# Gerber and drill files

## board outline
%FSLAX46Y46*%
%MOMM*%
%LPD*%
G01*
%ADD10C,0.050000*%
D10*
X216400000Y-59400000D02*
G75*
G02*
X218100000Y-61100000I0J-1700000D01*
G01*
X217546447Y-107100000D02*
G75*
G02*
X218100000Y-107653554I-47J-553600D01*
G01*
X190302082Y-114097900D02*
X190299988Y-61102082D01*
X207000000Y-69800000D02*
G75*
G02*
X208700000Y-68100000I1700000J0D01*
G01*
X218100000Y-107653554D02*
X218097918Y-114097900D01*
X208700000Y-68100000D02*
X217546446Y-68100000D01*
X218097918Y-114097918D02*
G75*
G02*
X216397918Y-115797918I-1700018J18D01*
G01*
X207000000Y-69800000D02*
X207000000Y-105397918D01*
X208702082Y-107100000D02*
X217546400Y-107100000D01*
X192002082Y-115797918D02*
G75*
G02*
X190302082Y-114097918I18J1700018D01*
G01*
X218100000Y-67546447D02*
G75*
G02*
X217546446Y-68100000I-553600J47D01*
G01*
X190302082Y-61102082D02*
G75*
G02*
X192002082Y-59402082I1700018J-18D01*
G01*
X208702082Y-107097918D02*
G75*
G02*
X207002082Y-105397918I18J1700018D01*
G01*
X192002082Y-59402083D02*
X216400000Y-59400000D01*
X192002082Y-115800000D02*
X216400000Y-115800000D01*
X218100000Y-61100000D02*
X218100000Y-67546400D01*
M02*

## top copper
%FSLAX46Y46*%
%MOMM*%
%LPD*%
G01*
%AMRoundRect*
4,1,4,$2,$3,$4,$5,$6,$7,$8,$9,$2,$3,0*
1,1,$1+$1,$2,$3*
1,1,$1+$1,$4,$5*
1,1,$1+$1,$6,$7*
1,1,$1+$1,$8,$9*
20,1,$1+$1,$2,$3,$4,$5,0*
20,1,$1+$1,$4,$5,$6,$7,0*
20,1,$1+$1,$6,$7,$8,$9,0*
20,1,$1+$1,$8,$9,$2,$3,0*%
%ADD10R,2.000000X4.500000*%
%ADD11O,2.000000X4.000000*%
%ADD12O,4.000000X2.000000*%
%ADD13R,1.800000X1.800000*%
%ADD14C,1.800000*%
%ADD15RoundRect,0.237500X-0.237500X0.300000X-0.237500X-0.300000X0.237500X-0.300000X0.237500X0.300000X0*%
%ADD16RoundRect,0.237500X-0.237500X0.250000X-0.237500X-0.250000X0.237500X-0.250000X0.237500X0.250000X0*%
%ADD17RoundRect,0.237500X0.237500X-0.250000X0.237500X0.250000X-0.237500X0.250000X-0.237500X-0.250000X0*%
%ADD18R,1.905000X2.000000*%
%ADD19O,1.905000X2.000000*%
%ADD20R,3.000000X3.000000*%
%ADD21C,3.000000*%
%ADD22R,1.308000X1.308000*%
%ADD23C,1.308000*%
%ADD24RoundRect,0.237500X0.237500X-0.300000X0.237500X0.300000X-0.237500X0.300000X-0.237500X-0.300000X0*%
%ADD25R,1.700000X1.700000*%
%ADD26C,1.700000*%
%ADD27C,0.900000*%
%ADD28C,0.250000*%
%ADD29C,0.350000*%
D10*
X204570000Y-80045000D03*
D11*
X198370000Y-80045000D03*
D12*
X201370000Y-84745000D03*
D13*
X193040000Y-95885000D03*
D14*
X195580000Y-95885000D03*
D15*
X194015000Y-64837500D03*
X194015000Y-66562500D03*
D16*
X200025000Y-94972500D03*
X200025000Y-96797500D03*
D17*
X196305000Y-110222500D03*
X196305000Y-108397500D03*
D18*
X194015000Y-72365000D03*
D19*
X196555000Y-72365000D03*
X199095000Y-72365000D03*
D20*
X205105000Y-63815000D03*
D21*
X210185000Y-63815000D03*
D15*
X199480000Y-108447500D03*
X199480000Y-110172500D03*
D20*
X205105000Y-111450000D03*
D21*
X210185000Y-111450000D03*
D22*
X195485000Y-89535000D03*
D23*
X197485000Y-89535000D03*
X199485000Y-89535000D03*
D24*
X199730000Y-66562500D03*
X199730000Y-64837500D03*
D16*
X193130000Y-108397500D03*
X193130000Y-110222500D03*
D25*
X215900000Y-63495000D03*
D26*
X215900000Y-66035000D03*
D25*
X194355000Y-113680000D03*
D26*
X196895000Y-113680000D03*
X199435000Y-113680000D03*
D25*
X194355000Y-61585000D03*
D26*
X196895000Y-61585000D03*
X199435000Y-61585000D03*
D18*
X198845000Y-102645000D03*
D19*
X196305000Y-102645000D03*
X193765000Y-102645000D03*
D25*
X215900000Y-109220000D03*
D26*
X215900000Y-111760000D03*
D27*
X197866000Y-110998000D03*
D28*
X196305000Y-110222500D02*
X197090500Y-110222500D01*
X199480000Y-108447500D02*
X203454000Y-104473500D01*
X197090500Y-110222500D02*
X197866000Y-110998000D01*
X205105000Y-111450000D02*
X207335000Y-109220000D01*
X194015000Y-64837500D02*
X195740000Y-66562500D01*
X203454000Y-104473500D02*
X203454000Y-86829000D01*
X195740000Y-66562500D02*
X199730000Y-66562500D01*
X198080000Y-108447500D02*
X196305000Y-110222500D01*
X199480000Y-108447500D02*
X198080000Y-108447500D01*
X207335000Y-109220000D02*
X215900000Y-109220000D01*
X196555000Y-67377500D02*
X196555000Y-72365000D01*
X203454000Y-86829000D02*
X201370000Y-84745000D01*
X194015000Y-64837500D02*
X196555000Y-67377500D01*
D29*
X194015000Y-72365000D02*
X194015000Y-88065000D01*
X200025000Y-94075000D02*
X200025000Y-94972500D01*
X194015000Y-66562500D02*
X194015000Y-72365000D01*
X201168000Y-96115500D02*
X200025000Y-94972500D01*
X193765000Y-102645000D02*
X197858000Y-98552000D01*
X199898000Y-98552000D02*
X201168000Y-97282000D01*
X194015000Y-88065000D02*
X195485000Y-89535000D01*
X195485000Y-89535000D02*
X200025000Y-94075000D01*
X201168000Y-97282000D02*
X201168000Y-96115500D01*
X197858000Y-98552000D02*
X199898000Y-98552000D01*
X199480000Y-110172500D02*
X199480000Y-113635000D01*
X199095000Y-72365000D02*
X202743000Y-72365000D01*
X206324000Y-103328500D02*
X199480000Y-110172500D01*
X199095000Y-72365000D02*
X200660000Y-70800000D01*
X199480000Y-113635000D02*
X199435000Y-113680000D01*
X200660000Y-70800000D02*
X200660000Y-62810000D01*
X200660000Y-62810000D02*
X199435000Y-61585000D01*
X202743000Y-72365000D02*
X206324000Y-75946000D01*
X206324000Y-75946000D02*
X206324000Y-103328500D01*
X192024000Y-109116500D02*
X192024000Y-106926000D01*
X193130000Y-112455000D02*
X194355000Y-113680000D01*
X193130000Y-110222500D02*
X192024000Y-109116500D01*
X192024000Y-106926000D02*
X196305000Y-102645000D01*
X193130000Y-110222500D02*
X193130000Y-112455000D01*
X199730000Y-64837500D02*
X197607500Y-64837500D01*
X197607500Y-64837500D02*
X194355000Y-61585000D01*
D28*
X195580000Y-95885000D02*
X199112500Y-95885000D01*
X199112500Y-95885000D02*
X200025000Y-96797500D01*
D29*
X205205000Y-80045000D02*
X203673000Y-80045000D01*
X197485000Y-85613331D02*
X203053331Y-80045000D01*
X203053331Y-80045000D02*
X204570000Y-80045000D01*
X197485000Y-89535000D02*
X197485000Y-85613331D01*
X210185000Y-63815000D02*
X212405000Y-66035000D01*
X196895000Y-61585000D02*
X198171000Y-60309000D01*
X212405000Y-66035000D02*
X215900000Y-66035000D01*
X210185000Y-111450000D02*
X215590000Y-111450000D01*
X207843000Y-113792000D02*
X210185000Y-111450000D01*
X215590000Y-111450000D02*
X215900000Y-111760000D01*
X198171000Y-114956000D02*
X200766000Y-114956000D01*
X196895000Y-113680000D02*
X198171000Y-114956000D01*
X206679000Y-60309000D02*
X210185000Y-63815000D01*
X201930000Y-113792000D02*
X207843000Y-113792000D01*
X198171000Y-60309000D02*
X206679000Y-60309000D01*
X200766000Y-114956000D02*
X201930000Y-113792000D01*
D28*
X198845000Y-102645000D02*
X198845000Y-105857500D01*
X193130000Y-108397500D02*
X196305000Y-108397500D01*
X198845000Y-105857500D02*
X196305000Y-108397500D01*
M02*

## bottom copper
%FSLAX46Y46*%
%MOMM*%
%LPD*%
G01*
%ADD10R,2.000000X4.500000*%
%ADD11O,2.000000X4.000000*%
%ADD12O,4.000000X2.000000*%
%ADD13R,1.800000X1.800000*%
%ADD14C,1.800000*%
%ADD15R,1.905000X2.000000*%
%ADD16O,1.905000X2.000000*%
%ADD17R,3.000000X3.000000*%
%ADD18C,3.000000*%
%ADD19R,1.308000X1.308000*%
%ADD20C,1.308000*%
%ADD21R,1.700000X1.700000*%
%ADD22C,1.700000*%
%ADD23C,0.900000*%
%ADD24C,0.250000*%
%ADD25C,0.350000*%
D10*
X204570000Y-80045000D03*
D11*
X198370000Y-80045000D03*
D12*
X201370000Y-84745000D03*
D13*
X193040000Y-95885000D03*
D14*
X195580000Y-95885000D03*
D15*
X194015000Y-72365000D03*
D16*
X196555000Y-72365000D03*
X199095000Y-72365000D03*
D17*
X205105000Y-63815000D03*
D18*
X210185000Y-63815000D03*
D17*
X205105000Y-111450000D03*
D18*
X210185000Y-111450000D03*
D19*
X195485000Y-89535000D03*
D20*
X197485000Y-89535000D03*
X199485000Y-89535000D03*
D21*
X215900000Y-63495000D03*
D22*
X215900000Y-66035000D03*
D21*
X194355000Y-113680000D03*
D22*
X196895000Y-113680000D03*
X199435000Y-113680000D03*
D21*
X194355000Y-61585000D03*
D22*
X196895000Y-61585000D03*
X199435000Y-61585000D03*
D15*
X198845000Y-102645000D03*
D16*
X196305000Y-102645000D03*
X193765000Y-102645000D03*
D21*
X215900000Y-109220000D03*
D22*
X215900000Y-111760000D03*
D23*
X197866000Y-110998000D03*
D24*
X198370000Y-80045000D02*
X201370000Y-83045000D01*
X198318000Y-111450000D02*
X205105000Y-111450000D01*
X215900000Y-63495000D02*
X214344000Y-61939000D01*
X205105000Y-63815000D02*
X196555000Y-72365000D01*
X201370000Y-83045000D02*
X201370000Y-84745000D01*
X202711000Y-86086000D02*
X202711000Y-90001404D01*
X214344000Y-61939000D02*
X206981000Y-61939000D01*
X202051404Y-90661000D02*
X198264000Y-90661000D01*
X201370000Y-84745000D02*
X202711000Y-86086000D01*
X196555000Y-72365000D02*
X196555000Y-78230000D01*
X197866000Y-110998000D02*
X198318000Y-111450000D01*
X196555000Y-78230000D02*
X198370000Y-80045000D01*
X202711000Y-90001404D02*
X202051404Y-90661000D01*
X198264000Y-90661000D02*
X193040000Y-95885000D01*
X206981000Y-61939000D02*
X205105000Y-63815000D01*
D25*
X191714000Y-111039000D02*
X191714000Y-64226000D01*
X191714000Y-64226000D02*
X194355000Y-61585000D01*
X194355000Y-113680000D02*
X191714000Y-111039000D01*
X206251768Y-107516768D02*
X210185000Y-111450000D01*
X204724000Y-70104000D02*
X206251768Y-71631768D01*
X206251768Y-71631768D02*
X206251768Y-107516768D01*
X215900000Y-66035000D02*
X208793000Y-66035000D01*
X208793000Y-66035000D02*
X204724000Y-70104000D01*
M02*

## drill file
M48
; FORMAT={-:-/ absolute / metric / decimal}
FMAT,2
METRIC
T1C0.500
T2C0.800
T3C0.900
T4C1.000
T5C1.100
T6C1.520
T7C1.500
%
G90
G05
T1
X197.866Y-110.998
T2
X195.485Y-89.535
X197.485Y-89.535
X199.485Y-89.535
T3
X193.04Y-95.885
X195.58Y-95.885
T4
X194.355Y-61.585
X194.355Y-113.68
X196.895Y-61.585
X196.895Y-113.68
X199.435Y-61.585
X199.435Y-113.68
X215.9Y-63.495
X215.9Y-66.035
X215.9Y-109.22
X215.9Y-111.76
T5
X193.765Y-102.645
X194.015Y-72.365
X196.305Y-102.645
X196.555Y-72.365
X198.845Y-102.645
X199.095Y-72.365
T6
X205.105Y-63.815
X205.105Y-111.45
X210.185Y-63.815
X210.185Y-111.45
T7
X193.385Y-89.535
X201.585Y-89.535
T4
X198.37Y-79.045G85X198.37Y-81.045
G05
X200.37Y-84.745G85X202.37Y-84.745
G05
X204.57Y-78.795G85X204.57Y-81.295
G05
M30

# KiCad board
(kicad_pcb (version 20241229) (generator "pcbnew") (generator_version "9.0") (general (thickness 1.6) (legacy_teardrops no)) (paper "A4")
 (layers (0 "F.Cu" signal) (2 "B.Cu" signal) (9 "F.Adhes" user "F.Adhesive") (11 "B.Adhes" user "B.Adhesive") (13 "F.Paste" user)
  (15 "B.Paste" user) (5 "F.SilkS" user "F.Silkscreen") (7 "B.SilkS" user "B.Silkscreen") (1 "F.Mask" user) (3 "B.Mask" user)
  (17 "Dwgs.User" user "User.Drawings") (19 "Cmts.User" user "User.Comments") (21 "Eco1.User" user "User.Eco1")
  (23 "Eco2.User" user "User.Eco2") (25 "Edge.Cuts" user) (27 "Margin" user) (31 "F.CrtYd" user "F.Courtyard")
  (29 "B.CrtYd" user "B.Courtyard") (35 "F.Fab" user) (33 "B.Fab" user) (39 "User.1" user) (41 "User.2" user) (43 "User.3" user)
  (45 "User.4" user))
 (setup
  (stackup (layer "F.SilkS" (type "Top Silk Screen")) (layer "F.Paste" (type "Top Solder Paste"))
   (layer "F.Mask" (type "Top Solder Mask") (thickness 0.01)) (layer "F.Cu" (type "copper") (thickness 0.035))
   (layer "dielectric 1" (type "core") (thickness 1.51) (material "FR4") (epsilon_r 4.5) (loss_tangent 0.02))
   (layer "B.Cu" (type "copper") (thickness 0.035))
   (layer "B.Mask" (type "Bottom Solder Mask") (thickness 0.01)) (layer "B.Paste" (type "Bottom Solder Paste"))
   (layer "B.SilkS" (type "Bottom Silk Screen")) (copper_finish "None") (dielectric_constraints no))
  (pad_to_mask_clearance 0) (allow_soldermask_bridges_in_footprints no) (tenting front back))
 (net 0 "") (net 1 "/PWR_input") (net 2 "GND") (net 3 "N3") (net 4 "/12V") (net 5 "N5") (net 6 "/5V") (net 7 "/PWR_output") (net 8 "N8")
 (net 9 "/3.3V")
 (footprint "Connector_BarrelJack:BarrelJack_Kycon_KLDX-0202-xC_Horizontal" (layer "F.Cu") (at 204.57 80.045)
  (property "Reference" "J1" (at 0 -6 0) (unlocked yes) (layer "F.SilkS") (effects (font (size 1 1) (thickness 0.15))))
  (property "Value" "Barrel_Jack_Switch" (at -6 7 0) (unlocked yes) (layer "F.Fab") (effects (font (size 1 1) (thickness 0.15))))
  (pad "1" thru_hole rect (at 0 0) (size 2 4.5) (drill oval 1 3.5) (layers "*.Cu" "*.Mask") (remove_unused_layers no) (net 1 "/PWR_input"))
  (pad "2" thru_hole oval (at -6.2 0) (size 2 4) (drill oval 1 3) (layers "*.Cu" "*.Mask") (remove_unused_layers no) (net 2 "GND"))
  (pad "3" thru_hole oval (at -3.2 4.7 90) (size 2 4) (drill oval 1 3) (layers "*.Cu" "*.Mask") (remove_unused_layers no) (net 2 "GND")))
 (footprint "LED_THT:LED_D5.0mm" (layer "F.Cu") (at 193.04 95.885)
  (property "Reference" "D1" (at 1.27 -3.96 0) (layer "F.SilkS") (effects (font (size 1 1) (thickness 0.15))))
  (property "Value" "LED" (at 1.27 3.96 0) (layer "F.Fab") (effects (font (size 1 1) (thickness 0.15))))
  (pad "1" thru_hole rect (at 0 0) (size 1.8 1.8) (drill 0.9) (layers "*.Cu" "*.Mask") (remove_unused_layers no) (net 2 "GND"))
  (pad "2" thru_hole circle (at 2.54 0) (size 1.8 1.8) (drill 0.9) (layers "*.Cu" "*.Mask") (remove_unused_layers no) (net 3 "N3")))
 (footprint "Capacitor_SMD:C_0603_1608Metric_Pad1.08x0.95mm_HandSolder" (layer "F.Cu") (at 194.015 65.7 -90)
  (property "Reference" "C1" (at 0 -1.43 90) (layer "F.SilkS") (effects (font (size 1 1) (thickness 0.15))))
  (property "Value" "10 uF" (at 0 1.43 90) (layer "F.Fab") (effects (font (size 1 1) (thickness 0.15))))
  (pad "1" smd roundrect (at -0.8625 0 270) (size 1.075 0.95) (layers "F.Cu" "F.Mask" "F.Paste") (roundrect_rratio 0.25) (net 2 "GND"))
  (pad "2" smd roundrect (at 0.8625 0 270) (size 1.075 0.95) (layers "F.Cu" "F.Mask" "F.Paste") (roundrect_rratio 0.25) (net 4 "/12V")))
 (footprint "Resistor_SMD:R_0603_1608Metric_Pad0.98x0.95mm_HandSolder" (layer "F.Cu") (at 200.025 95.885 -90)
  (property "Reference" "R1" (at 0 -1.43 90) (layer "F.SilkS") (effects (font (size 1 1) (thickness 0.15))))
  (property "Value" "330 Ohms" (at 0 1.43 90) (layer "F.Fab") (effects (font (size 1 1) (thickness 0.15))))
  (pad "1" smd roundrect (at -0.9125 0 270) (size 0.975 0.95) (layers "F.Cu" "F.Mask" "F.Paste") (roundrect_rratio 0.25) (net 4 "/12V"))
  (pad "2" smd roundrect (at 0.9125 0 270) (size 0.975 0.95) (layers "F.Cu" "F.Mask" "F.Paste") (roundrect_rratio 0.25) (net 3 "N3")))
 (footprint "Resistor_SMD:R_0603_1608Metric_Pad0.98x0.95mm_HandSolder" (layer "F.Cu") (at 196.305 109.31 90)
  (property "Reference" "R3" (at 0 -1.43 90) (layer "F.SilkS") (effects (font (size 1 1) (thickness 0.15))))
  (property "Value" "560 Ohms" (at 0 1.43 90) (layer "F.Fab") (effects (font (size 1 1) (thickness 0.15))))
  (pad "1" smd roundrect (at -0.9125 0 90) (size 0.975 0.95) (layers "F.Cu" "F.Mask" "F.Paste") (roundrect_rratio 0.25) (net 2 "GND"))
  (pad "2" smd roundrect (at 0.9125 0 90) (size 0.975 0.95) (layers "F.Cu" "F.Mask" "F.Paste") (roundrect_rratio 0.25) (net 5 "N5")))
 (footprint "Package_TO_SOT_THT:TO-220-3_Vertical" (layer "F.Cu") (at 194.015 72.365)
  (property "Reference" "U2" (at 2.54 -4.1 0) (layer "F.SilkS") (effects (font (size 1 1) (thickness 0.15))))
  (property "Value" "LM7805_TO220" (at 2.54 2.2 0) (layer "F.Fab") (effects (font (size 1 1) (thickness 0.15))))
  (pad "1" thru_hole rect (at 0 0) (size 1.905 2) (drill 1.1) (layers "*.Cu" "*.Mask") (remove_unused_layers no) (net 4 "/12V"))
  (pad "2" thru_hole oval (at 2.54 0) (size 1.905 2) (drill 1.1) (layers "*.Cu" "*.Mask") (remove_unused_layers no) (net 2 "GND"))
  (pad "3" thru_hole oval (at 5.08 0) (size 1.905 2) (drill 1.1) (layers "*.Cu" "*.Mask") (remove_unused_layers no) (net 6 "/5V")))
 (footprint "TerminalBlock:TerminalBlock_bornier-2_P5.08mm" (layer "F.Cu") (at 205.105 63.815)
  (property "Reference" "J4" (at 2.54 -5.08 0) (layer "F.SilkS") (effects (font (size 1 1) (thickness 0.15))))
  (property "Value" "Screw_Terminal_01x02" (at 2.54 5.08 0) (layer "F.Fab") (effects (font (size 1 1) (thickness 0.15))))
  (pad "1" thru_hole rect (at 0 0) (size 3 3) (drill 1.52) (layers "*.Cu" "*.Mask") (remove_unused_layers no) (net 2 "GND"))
  (pad "2" thru_hole circle (at 5.08 0) (size 3 3) (drill 1.52) (layers "*.Cu" "*.Mask") (remove_unused_layers no) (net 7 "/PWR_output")))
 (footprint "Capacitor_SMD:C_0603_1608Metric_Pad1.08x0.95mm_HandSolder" (layer "F.Cu") (at 199.48 109.31 -90)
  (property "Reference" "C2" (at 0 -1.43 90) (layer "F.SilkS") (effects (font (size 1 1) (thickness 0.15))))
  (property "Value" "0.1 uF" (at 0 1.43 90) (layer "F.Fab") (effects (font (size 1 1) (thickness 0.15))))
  (pad "1" smd roundrect (at -0.8625 0 270) (size 1.075 0.95) (layers "F.Cu" "F.Mask" "F.Paste") (roundrect_rratio 0.25) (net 2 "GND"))
  (pad "2" smd roundrect (at 0.8625 0 270) (size 1.075 0.95) (layers "F.Cu" "F.Mask" "F.Paste") (roundrect_rratio 0.25) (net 6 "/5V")))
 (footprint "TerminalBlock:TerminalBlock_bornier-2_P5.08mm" (layer "F.Cu") (at 205.105 111.45)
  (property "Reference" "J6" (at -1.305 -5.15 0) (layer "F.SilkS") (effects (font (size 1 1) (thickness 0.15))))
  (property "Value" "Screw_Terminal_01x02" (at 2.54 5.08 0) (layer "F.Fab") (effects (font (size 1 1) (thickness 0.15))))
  (pad "1" thru_hole rect (at 0 0) (size 3 3) (drill 1.52) (layers "*.Cu" "*.Mask") (remove_unused_layers no) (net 2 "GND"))
  (pad "2" thru_hole circle (at 5.08 0) (size 3 3) (drill 1.52) (layers "*.Cu" "*.Mask") (remove_unused_layers no) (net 7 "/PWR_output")))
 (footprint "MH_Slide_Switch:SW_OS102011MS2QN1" (layer "F.Cu") (at 197.485 89.535)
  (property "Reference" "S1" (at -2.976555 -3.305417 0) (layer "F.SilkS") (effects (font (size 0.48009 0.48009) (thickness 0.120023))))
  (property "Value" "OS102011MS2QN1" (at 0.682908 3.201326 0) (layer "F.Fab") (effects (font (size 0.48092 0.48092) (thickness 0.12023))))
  (pad "" np_thru_hole circle (at -4.1 0) (size 1.5 1.5) (drill 1.5) (layers "*.Cu" "*.Mask"))
  (pad "" np_thru_hole circle (at 4.1 0) (size 1.5 1.5) (drill 1.5) (layers "*.Cu" "*.Mask"))
  (pad "1" thru_hole rect (at -2 0) (size 1.308 1.308) (drill 0.8) (layers "*.Cu" "*.Mask") (remove_unused_layers no) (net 4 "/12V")
   (solder_mask_margin 0.102))
  (pad "2" thru_hole circle (at 0 0) (size 1.308 1.308) (drill 0.8) (layers "*.Cu" "*.Mask") (remove_unused_layers no) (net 1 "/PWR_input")
   (solder_mask_margin 0.102))
  (pad "3" thru_hole circle (at 2 0) (size 1.308 1.308) (drill 0.8) (layers "*.Cu" "*.Mask") (remove_unused_layers no) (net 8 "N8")
   (solder_mask_margin 0.102)))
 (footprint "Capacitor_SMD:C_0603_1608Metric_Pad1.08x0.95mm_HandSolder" (layer "F.Cu") (at 199.73 65.7 90)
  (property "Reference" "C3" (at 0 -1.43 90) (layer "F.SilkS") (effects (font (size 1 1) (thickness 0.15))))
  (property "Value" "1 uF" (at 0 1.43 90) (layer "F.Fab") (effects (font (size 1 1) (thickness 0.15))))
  (pad "1" smd roundrect (at -0.8625 0 90) (size 1.075 0.95) (layers "F.Cu" "F.Mask" "F.Paste") (roundrect_rratio 0.25) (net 2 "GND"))
  (pad "2" smd roundrect (at 0.8625 0 90) (size 1.075 0.95) (layers "F.Cu" "F.Mask" "F.Paste") (roundrect_rratio 0.25) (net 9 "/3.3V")))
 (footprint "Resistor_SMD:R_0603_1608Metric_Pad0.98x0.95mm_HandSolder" (layer "F.Cu") (at 193.13 109.31 -90)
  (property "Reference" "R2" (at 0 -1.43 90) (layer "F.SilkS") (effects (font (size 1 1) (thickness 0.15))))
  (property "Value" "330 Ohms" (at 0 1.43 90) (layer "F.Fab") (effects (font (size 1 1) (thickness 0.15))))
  (pad "1" smd roundrect (at -0.9125 0 270) (size 0.975 0.95) (layers "F.Cu" "F.Mask" "F.Paste") (roundrect_rratio 0.25) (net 5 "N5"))
  (pad "2" smd roundrect (at 0.9125 0 270) (size 0.975 0.95) (layers "F.Cu" "F.Mask" "F.Paste") (roundrect_rratio 0.25) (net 9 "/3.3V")))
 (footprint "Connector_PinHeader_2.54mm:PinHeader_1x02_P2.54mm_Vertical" (layer "F.Cu") (at 215.9 63.495)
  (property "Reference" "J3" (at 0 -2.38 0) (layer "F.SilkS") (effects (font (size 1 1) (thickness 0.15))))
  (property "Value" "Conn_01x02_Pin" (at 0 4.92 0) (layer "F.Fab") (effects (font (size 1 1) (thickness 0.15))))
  (pad "1" thru_hole rect (at 0 0) (size 1.7 1.7) (drill 1) (layers "*.Cu" "*.Mask") (remove_unused_layers no) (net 2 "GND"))
  (pad "2" thru_hole circle (at 0 2.54) (size 1.7 1.7) (drill 1) (layers "*.Cu" "*.Mask") (remove_unused_layers no) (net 7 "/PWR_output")))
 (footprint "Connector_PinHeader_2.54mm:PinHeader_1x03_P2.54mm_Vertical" (layer "F.Cu") (at 194.355 113.68 90)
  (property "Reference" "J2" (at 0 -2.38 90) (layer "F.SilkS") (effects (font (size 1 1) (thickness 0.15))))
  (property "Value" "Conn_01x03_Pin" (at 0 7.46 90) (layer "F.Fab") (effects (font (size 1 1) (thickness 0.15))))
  (pad "1" thru_hole rect (at 0 0 90) (size 1.7 1.7) (drill 1) (layers "*.Cu" "*.Mask") (remove_unused_layers no) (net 9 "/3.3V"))
  (pad "2" thru_hole circle (at 0 2.54 90) (size 1.7 1.7) (drill 1) (layers "*.Cu" "*.Mask") (remove_unused_layers no) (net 7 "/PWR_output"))
  (pad "3" thru_hole circle (at 0 5.08 90) (size 1.7 1.7) (drill 1) (layers "*.Cu" "*.Mask") (remove_unused_layers no) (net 6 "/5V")))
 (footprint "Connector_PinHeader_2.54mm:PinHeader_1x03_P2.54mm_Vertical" (layer "F.Cu") (at 194.355 61.585 90)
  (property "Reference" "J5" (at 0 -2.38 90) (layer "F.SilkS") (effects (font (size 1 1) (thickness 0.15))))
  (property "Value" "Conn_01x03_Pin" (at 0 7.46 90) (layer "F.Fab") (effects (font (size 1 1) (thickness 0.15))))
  (pad "1" thru_hole rect (at 0 0 90) (size 1.7 1.7) (drill 1) (layers "*.Cu" "*.Mask") (remove_unused_layers no) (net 9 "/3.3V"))
  (pad "2" thru_hole circle (at 0 2.54 90) (size 1.7 1.7) (drill 1) (layers "*.Cu" "*.Mask") (remove_unused_layers no) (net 7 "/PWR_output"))
  (pad "3" thru_hole circle (at 0 5.08 90) (size 1.7 1.7) (drill 1) (layers "*.Cu" "*.Mask") (remove_unused_layers no) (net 6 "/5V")))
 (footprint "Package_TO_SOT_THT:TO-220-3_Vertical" (layer "F.Cu") (at 198.845 102.645 180)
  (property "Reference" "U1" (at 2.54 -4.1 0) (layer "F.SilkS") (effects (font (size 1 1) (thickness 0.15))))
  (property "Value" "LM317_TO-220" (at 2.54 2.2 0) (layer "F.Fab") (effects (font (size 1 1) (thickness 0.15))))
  (pad "1" thru_hole rect (at 0 0 180) (size 1.905 2) (drill 1.1) (layers "*.Cu" "*.Mask") (remove_unused_layers no) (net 5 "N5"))
  (pad "2" thru_hole oval (at 2.54 0 180) (size 1.905 2) (drill 1.1) (layers "*.Cu" "*.Mask") (remove_unused_layers no) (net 9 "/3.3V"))
  (pad "3" thru_hole oval (at 5.08 0 180) (size 1.905 2) (drill 1.1) (layers "*.Cu" "*.Mask") (remove_unused_layers no) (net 4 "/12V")))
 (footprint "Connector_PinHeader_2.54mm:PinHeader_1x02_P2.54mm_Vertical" (layer "F.Cu") (at 215.9 109.22)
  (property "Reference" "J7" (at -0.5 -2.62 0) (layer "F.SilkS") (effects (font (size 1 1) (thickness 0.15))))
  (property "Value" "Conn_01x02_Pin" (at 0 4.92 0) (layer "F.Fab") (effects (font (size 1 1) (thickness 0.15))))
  (pad "1" thru_hole rect (at 0 0) (size 1.7 1.7) (drill 1) (layers "*.Cu" "*.Mask") (remove_unused_layers no) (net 2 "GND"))
  (pad "2" thru_hole circle (at 0 2.54) (size 1.7 1.7) (drill 1) (layers "*.Cu" "*.Mask") (remove_unused_layers no) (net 7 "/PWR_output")))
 (gr_arc (start 216.4 59.4) (mid 217.602082 59.897918) (end 218.1 61.1) (stroke (width 0.05) (type default)) (layer "Edge.Cuts"))
 (gr_arc (start 217.546447 107.1) (mid 217.937869 107.262132) (end 218.1 107.653554) (stroke (width 0.05) (type default))
  (layer "Edge.Cuts"))
 (gr_line (start 190.302082 114.0979) (end 190.299988 61.102082) (stroke (width 0.05) (type default)) (layer "Edge.Cuts"))
 (gr_arc (start 207 69.8) (mid 207.497918 68.597918) (end 208.7 68.1) (stroke (width 0.05) (type default)) (layer "Edge.Cuts"))
 (gr_line (start 218.1 107.653554) (end 218.097918 114.0979) (stroke (width 0.05) (type default)) (layer "Edge.Cuts"))
 (gr_line (start 208.7 68.1) (end 217.546446 68.1) (stroke (width 0.05) (type default)) (layer "Edge.Cuts"))
 (gr_arc (start 218.097918 114.097918) (mid 217.6 115.3) (end 216.397918 115.797918) (stroke (width 0.05) (type default))
  (layer "Edge.Cuts"))
 (gr_line (start 207 69.8) (end 207 105.397918) (stroke (width 0.05) (type default)) (layer "Edge.Cuts"))
 (gr_line (start 208.702082 107.1) (end 217.5464 107.1) (stroke (width 0.05) (type default)) (layer "Edge.Cuts"))
 (gr_arc (start 192.002082 115.797918) (mid 190.8 115.3) (end 190.302082 114.097918) (stroke (width 0.05) (type default))
  (layer "Edge.Cuts"))
 (gr_arc (start 218.1 67.546447) (mid 217.937868 67.937869) (end 217.546446 68.1) (stroke (width 0.05) (type default)) (layer "Edge.Cuts"))
 (gr_arc (start 190.302082 61.102082) (mid 190.8 59.9) (end 192.002082 59.402082) (stroke (width 0.05) (type default)) (layer "Edge.Cuts"))
 (gr_arc (start 208.702082 107.097918) (mid 207.5 106.6) (end 207.002082 105.397918) (stroke (width 0.05) (type default))
  (layer "Edge.Cuts"))
 (gr_line (start 192.002082 59.402083) (end 216.4 59.4) (stroke (width 0.05) (type default)) (layer "Edge.Cuts"))
 (gr_line (start 192.002082 115.8) (end 216.4 115.8) (stroke (width 0.05) (type default)) (layer "Edge.Cuts"))
 (gr_line (start 218.1 61.1) (end 218.1 67.5464) (stroke (width 0.05) (type default)) (layer "Edge.Cuts"))
 (segment (start 196.305 110.2225) (end 197.0905 110.2225) (width 0.25) (layer "F.Cu") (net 2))
 (segment (start 199.48 108.4475) (end 203.454 104.4735) (width 0.25) (layer "F.Cu") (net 2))
 (segment (start 197.0905 110.2225) (end 197.866 110.998) (width 0.25) (layer "F.Cu") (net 2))
 (segment (start 205.105 111.45) (end 207.335 109.22) (width 0.25) (layer "F.Cu") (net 2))
 (segment (start 194.015 64.8375) (end 195.74 66.5625) (width 0.25) (layer "F.Cu") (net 2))
 (segment (start 203.454 104.4735) (end 203.454 86.829) (width 0.25) (layer "F.Cu") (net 2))
 (segment (start 195.74 66.5625) (end 199.73 66.5625) (width 0.25) (layer "F.Cu") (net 2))
 (segment (start 198.08 108.4475) (end 196.305 110.2225) (width 0.25) (layer "F.Cu") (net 2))
 (segment (start 199.48 108.4475) (end 198.08 108.4475) (width 0.25) (layer "F.Cu") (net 2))
 (segment (start 207.335 109.22) (end 215.9 109.22) (width 0.25) (layer "F.Cu") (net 2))
 (segment (start 196.555 67.3775) (end 196.555 72.365) (width 0.25) (layer "F.Cu") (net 2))
 (segment (start 203.454 86.829) (end 201.37 84.745) (width 0.25) (layer "F.Cu") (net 2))
 (segment (start 194.015 64.8375) (end 196.555 67.3775) (width 0.25) (layer "F.Cu") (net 2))
 (via (at 197.866 110.998) (size 0.9) (drill 0.5) (layers "F.Cu" "B.Cu") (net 2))
 (segment (start 198.37 80.045) (end 201.37 83.045) (width 0.25) (layer "B.Cu") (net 2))
 (segment (start 198.318 111.45) (end 205.105 111.45) (width 0.25) (layer "B.Cu") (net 2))
 (segment (start 215.9 63.495) (end 214.344 61.939) (width 0.25) (layer "B.Cu") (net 2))
 (segment (start 205.105 63.815) (end 196.555 72.365) (width 0.25) (layer "B.Cu") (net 2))
 (segment (start 201.37 83.045) (end 201.37 84.745) (width 0.25) (layer "B.Cu") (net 2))
 (segment (start 202.711 86.086) (end 202.711 90.001404) (width 0.25) (layer "B.Cu") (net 2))
 (segment (start 214.344 61.939) (end 206.981 61.939) (width 0.25) (layer "B.Cu") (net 2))
 (segment (start 202.051404 90.661) (end 198.264 90.661) (width 0.25) (layer "B.Cu") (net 2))
 (segment (start 201.37 84.745) (end 202.711 86.086) (width 0.25) (layer "B.Cu") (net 2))
 (segment (start 196.555 72.365) (end 196.555 78.23) (width 0.25) (layer "B.Cu") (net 2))
 (segment (start 197.866 110.998) (end 198.318 111.45) (width 0.25) (layer "B.Cu") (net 2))
 (segment (start 196.555 78.23) (end 198.37 80.045) (width 0.25) (layer "B.Cu") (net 2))
 (segment (start 202.711 90.001404) (end 202.051404 90.661) (width 0.25) (layer "B.Cu") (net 2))
 (segment (start 198.264 90.661) (end 193.04 95.885) (width 0.25) (layer "B.Cu") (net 2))
 (segment (start 206.981 61.939) (end 205.105 63.815) (width 0.25) (layer "B.Cu") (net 2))
 (segment (start 194.015 72.365) (end 194.015 88.065) (width 0.35) (layer "F.Cu") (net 4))
 (segment (start 200.025 94.075) (end 200.025 94.9725) (width 0.35) (layer "F.Cu") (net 4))
 (segment (start 194.015 66.5625) (end 194.015 72.365) (width 0.35) (layer "F.Cu") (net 4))
 (segment (start 201.168 96.1155) (end 200.025 94.9725) (width 0.35) (layer "F.Cu") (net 4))
 (segment (start 193.765 102.645) (end 197.858 98.552) (width 0.35) (layer "F.Cu") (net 4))
 (segment (start 199.898 98.552) (end 201.168 97.282) (width 0.35) (layer "F.Cu") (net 4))
 (segment (start 194.015 88.065) (end 195.485 89.535) (width 0.35) (layer "F.Cu") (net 4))
 (segment (start 195.485 89.535) (end 200.025 94.075) (width 0.35) (layer "F.Cu") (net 4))
 (segment (start 201.168 97.282) (end 201.168 96.1155) (width 0.35) (layer "F.Cu") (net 4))
 (segment (start 197.858 98.552) (end 199.898 98.552) (width 0.35) (layer "F.Cu") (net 4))
 (segment (start 199.48 110.1725) (end 199.48 113.635) (width 0.35) (layer "F.Cu") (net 6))
 (segment (start 199.095 72.365) (end 202.743 72.365) (width 0.35) (layer "F.Cu") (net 6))
 (segment (start 206.324 103.3285) (end 199.48 110.1725) (width 0.35) (layer "F.Cu") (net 6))
 (segment (start 199.095 72.365) (end 200.66 70.8) (width 0.35) (layer "F.Cu") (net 6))
 (segment (start 199.48 113.635) (end 199.435 113.68) (width 0.35) (layer "F.Cu") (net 6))
 (segment (start 200.66 70.8) (end 200.66 62.81) (width 0.35) (layer "F.Cu") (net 6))
 (segment (start 200.66 62.81) (end 199.435 61.585) (width 0.35) (layer "F.Cu") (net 6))
 (segment (start 202.743 72.365) (end 206.324 75.946) (width 0.35) (layer "F.Cu") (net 6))
 (segment (start 206.324 75.946) (end 206.324 103.3285) (width 0.35) (layer "F.Cu") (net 6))
 (segment (start 192.024 109.1165) (end 192.024 106.926) (width 0.35) (layer "F.Cu") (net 9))
 (segment (start 193.13 112.455) (end 194.355 113.68) (width 0.35) (layer "F.Cu") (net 9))
 (segment (start 193.13 110.2225) (end 192.024 109.1165) (width 0.35) (layer "F.Cu") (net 9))
 (segment (start 192.024 106.926) (end 196.305 102.645) (width 0.35) (layer "F.Cu") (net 9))
 (segment (start 193.13 110.2225) (end 193.13 112.455) (width 0.35) (layer "F.Cu") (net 9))
 (segment (start 199.73 64.8375) (end 197.6075 64.8375) (width 0.35) (layer "F.Cu") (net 9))
 (segment (start 197.6075 64.8375) (end 194.355 61.585) (width 0.35) (layer "F.Cu") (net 9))
 (segment (start 191.714 111.039) (end 191.714 64.226) (width 0.35) (layer "B.Cu") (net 9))
 (segment (start 191.714 64.226) (end 194.355 61.585) (width 0.35) (layer "B.Cu") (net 9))
 (segment (start 194.355 113.68) (end 191.714 111.039) (width 0.35) (layer "B.Cu") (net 9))
 (segment (start 195.58 95.885) (end 199.1125 95.885) (width 0.25) (layer "F.Cu") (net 3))
 (segment (start 199.1125 95.885) (end 200.025 96.7975) (width 0.25) (layer "F.Cu") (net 3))
 (segment (start 205.205 80.045) (end 203.673 80.045) (width 0.35) (layer "F.Cu") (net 1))
 (segment (start 197.485 85.613331) (end 203.053331 80.045) (width 0.35) (layer "F.Cu") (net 1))
 (segment (start 203.053331 80.045) (end 204.57 80.045) (width 0.35) (layer "F.Cu") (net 1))
 (segment (start 197.485 89.535) (end 197.485 85.613331) (width 0.35) (layer "F.Cu") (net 1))
 (segment (start 210.185 63.815) (end 212.405 66.035) (width 0.35) (layer "F.Cu") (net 7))
 (segment (start 196.895 61.585) (end 198.171 60.309) (width 0.35) (layer "F.Cu") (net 7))
 (segment (start 212.405 66.035) (end 215.9 66.035) (width 0.35) (layer "F.Cu") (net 7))
 (segment (start 210.185 111.45) (end 215.59 111.45) (width 0.35) (layer "F.Cu") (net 7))
 (segment (start 207.843 113.792) (end 210.185 111.45) (width 0.35) (layer "F.Cu") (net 7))
 (segment (start 215.59 111.45) (end 215.9 111.76) (width 0.35) (layer "F.Cu") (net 7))
 (segment (start 198.171 114.956) (end 200.766 114.956) (width 0.35) (layer "F.Cu") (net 7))
 (segment (start 196.895 113.68) (end 198.171 114.956) (width 0.35) (layer "F.Cu") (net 7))
 (segment (start 206.679 60.309) (end 210.185 63.815) (width 0.35) (layer "F.Cu") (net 7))
 (segment (start 201.93 113.792) (end 207.843 113.792) (width 0.35) (layer "F.Cu") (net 7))
 (segment (start 198.171 60.309) (end 206.679 60.309) (width 0.35) (layer "F.Cu") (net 7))
 (segment (start 200.766 114.956) (end 201.93 113.792) (width 0.35) (layer "F.Cu") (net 7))
 (segment (start 206.251768 107.516768) (end 210.185 111.45) (width 0.35) (layer "B.Cu") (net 7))
 (segment (start 204.724 70.104) (end 206.251768 71.631768) (width 0.35) (layer "B.Cu") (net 7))
 (segment (start 206.251768 71.631768) (end 206.251768 107.516768) (width 0.35) (layer "B.Cu") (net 7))
 (segment (start 215.9 66.035) (end 208.793 66.035) (width 0.35) (layer "B.Cu") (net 7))
 (segment (start 208.793 66.035) (end 204.724 70.104) (width 0.35) (layer "B.Cu") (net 7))
 (segment (start 198.845 102.645) (end 198.845 105.8575) (width 0.25) (layer "F.Cu") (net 5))
 (segment (start 193.13 108.3975) (end 196.305 108.3975) (width 0.25) (layer "F.Cu") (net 5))
 (segment (start 198.845 105.8575) (end 196.305 108.3975) (width 0.25) (layer "F.Cu") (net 5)))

